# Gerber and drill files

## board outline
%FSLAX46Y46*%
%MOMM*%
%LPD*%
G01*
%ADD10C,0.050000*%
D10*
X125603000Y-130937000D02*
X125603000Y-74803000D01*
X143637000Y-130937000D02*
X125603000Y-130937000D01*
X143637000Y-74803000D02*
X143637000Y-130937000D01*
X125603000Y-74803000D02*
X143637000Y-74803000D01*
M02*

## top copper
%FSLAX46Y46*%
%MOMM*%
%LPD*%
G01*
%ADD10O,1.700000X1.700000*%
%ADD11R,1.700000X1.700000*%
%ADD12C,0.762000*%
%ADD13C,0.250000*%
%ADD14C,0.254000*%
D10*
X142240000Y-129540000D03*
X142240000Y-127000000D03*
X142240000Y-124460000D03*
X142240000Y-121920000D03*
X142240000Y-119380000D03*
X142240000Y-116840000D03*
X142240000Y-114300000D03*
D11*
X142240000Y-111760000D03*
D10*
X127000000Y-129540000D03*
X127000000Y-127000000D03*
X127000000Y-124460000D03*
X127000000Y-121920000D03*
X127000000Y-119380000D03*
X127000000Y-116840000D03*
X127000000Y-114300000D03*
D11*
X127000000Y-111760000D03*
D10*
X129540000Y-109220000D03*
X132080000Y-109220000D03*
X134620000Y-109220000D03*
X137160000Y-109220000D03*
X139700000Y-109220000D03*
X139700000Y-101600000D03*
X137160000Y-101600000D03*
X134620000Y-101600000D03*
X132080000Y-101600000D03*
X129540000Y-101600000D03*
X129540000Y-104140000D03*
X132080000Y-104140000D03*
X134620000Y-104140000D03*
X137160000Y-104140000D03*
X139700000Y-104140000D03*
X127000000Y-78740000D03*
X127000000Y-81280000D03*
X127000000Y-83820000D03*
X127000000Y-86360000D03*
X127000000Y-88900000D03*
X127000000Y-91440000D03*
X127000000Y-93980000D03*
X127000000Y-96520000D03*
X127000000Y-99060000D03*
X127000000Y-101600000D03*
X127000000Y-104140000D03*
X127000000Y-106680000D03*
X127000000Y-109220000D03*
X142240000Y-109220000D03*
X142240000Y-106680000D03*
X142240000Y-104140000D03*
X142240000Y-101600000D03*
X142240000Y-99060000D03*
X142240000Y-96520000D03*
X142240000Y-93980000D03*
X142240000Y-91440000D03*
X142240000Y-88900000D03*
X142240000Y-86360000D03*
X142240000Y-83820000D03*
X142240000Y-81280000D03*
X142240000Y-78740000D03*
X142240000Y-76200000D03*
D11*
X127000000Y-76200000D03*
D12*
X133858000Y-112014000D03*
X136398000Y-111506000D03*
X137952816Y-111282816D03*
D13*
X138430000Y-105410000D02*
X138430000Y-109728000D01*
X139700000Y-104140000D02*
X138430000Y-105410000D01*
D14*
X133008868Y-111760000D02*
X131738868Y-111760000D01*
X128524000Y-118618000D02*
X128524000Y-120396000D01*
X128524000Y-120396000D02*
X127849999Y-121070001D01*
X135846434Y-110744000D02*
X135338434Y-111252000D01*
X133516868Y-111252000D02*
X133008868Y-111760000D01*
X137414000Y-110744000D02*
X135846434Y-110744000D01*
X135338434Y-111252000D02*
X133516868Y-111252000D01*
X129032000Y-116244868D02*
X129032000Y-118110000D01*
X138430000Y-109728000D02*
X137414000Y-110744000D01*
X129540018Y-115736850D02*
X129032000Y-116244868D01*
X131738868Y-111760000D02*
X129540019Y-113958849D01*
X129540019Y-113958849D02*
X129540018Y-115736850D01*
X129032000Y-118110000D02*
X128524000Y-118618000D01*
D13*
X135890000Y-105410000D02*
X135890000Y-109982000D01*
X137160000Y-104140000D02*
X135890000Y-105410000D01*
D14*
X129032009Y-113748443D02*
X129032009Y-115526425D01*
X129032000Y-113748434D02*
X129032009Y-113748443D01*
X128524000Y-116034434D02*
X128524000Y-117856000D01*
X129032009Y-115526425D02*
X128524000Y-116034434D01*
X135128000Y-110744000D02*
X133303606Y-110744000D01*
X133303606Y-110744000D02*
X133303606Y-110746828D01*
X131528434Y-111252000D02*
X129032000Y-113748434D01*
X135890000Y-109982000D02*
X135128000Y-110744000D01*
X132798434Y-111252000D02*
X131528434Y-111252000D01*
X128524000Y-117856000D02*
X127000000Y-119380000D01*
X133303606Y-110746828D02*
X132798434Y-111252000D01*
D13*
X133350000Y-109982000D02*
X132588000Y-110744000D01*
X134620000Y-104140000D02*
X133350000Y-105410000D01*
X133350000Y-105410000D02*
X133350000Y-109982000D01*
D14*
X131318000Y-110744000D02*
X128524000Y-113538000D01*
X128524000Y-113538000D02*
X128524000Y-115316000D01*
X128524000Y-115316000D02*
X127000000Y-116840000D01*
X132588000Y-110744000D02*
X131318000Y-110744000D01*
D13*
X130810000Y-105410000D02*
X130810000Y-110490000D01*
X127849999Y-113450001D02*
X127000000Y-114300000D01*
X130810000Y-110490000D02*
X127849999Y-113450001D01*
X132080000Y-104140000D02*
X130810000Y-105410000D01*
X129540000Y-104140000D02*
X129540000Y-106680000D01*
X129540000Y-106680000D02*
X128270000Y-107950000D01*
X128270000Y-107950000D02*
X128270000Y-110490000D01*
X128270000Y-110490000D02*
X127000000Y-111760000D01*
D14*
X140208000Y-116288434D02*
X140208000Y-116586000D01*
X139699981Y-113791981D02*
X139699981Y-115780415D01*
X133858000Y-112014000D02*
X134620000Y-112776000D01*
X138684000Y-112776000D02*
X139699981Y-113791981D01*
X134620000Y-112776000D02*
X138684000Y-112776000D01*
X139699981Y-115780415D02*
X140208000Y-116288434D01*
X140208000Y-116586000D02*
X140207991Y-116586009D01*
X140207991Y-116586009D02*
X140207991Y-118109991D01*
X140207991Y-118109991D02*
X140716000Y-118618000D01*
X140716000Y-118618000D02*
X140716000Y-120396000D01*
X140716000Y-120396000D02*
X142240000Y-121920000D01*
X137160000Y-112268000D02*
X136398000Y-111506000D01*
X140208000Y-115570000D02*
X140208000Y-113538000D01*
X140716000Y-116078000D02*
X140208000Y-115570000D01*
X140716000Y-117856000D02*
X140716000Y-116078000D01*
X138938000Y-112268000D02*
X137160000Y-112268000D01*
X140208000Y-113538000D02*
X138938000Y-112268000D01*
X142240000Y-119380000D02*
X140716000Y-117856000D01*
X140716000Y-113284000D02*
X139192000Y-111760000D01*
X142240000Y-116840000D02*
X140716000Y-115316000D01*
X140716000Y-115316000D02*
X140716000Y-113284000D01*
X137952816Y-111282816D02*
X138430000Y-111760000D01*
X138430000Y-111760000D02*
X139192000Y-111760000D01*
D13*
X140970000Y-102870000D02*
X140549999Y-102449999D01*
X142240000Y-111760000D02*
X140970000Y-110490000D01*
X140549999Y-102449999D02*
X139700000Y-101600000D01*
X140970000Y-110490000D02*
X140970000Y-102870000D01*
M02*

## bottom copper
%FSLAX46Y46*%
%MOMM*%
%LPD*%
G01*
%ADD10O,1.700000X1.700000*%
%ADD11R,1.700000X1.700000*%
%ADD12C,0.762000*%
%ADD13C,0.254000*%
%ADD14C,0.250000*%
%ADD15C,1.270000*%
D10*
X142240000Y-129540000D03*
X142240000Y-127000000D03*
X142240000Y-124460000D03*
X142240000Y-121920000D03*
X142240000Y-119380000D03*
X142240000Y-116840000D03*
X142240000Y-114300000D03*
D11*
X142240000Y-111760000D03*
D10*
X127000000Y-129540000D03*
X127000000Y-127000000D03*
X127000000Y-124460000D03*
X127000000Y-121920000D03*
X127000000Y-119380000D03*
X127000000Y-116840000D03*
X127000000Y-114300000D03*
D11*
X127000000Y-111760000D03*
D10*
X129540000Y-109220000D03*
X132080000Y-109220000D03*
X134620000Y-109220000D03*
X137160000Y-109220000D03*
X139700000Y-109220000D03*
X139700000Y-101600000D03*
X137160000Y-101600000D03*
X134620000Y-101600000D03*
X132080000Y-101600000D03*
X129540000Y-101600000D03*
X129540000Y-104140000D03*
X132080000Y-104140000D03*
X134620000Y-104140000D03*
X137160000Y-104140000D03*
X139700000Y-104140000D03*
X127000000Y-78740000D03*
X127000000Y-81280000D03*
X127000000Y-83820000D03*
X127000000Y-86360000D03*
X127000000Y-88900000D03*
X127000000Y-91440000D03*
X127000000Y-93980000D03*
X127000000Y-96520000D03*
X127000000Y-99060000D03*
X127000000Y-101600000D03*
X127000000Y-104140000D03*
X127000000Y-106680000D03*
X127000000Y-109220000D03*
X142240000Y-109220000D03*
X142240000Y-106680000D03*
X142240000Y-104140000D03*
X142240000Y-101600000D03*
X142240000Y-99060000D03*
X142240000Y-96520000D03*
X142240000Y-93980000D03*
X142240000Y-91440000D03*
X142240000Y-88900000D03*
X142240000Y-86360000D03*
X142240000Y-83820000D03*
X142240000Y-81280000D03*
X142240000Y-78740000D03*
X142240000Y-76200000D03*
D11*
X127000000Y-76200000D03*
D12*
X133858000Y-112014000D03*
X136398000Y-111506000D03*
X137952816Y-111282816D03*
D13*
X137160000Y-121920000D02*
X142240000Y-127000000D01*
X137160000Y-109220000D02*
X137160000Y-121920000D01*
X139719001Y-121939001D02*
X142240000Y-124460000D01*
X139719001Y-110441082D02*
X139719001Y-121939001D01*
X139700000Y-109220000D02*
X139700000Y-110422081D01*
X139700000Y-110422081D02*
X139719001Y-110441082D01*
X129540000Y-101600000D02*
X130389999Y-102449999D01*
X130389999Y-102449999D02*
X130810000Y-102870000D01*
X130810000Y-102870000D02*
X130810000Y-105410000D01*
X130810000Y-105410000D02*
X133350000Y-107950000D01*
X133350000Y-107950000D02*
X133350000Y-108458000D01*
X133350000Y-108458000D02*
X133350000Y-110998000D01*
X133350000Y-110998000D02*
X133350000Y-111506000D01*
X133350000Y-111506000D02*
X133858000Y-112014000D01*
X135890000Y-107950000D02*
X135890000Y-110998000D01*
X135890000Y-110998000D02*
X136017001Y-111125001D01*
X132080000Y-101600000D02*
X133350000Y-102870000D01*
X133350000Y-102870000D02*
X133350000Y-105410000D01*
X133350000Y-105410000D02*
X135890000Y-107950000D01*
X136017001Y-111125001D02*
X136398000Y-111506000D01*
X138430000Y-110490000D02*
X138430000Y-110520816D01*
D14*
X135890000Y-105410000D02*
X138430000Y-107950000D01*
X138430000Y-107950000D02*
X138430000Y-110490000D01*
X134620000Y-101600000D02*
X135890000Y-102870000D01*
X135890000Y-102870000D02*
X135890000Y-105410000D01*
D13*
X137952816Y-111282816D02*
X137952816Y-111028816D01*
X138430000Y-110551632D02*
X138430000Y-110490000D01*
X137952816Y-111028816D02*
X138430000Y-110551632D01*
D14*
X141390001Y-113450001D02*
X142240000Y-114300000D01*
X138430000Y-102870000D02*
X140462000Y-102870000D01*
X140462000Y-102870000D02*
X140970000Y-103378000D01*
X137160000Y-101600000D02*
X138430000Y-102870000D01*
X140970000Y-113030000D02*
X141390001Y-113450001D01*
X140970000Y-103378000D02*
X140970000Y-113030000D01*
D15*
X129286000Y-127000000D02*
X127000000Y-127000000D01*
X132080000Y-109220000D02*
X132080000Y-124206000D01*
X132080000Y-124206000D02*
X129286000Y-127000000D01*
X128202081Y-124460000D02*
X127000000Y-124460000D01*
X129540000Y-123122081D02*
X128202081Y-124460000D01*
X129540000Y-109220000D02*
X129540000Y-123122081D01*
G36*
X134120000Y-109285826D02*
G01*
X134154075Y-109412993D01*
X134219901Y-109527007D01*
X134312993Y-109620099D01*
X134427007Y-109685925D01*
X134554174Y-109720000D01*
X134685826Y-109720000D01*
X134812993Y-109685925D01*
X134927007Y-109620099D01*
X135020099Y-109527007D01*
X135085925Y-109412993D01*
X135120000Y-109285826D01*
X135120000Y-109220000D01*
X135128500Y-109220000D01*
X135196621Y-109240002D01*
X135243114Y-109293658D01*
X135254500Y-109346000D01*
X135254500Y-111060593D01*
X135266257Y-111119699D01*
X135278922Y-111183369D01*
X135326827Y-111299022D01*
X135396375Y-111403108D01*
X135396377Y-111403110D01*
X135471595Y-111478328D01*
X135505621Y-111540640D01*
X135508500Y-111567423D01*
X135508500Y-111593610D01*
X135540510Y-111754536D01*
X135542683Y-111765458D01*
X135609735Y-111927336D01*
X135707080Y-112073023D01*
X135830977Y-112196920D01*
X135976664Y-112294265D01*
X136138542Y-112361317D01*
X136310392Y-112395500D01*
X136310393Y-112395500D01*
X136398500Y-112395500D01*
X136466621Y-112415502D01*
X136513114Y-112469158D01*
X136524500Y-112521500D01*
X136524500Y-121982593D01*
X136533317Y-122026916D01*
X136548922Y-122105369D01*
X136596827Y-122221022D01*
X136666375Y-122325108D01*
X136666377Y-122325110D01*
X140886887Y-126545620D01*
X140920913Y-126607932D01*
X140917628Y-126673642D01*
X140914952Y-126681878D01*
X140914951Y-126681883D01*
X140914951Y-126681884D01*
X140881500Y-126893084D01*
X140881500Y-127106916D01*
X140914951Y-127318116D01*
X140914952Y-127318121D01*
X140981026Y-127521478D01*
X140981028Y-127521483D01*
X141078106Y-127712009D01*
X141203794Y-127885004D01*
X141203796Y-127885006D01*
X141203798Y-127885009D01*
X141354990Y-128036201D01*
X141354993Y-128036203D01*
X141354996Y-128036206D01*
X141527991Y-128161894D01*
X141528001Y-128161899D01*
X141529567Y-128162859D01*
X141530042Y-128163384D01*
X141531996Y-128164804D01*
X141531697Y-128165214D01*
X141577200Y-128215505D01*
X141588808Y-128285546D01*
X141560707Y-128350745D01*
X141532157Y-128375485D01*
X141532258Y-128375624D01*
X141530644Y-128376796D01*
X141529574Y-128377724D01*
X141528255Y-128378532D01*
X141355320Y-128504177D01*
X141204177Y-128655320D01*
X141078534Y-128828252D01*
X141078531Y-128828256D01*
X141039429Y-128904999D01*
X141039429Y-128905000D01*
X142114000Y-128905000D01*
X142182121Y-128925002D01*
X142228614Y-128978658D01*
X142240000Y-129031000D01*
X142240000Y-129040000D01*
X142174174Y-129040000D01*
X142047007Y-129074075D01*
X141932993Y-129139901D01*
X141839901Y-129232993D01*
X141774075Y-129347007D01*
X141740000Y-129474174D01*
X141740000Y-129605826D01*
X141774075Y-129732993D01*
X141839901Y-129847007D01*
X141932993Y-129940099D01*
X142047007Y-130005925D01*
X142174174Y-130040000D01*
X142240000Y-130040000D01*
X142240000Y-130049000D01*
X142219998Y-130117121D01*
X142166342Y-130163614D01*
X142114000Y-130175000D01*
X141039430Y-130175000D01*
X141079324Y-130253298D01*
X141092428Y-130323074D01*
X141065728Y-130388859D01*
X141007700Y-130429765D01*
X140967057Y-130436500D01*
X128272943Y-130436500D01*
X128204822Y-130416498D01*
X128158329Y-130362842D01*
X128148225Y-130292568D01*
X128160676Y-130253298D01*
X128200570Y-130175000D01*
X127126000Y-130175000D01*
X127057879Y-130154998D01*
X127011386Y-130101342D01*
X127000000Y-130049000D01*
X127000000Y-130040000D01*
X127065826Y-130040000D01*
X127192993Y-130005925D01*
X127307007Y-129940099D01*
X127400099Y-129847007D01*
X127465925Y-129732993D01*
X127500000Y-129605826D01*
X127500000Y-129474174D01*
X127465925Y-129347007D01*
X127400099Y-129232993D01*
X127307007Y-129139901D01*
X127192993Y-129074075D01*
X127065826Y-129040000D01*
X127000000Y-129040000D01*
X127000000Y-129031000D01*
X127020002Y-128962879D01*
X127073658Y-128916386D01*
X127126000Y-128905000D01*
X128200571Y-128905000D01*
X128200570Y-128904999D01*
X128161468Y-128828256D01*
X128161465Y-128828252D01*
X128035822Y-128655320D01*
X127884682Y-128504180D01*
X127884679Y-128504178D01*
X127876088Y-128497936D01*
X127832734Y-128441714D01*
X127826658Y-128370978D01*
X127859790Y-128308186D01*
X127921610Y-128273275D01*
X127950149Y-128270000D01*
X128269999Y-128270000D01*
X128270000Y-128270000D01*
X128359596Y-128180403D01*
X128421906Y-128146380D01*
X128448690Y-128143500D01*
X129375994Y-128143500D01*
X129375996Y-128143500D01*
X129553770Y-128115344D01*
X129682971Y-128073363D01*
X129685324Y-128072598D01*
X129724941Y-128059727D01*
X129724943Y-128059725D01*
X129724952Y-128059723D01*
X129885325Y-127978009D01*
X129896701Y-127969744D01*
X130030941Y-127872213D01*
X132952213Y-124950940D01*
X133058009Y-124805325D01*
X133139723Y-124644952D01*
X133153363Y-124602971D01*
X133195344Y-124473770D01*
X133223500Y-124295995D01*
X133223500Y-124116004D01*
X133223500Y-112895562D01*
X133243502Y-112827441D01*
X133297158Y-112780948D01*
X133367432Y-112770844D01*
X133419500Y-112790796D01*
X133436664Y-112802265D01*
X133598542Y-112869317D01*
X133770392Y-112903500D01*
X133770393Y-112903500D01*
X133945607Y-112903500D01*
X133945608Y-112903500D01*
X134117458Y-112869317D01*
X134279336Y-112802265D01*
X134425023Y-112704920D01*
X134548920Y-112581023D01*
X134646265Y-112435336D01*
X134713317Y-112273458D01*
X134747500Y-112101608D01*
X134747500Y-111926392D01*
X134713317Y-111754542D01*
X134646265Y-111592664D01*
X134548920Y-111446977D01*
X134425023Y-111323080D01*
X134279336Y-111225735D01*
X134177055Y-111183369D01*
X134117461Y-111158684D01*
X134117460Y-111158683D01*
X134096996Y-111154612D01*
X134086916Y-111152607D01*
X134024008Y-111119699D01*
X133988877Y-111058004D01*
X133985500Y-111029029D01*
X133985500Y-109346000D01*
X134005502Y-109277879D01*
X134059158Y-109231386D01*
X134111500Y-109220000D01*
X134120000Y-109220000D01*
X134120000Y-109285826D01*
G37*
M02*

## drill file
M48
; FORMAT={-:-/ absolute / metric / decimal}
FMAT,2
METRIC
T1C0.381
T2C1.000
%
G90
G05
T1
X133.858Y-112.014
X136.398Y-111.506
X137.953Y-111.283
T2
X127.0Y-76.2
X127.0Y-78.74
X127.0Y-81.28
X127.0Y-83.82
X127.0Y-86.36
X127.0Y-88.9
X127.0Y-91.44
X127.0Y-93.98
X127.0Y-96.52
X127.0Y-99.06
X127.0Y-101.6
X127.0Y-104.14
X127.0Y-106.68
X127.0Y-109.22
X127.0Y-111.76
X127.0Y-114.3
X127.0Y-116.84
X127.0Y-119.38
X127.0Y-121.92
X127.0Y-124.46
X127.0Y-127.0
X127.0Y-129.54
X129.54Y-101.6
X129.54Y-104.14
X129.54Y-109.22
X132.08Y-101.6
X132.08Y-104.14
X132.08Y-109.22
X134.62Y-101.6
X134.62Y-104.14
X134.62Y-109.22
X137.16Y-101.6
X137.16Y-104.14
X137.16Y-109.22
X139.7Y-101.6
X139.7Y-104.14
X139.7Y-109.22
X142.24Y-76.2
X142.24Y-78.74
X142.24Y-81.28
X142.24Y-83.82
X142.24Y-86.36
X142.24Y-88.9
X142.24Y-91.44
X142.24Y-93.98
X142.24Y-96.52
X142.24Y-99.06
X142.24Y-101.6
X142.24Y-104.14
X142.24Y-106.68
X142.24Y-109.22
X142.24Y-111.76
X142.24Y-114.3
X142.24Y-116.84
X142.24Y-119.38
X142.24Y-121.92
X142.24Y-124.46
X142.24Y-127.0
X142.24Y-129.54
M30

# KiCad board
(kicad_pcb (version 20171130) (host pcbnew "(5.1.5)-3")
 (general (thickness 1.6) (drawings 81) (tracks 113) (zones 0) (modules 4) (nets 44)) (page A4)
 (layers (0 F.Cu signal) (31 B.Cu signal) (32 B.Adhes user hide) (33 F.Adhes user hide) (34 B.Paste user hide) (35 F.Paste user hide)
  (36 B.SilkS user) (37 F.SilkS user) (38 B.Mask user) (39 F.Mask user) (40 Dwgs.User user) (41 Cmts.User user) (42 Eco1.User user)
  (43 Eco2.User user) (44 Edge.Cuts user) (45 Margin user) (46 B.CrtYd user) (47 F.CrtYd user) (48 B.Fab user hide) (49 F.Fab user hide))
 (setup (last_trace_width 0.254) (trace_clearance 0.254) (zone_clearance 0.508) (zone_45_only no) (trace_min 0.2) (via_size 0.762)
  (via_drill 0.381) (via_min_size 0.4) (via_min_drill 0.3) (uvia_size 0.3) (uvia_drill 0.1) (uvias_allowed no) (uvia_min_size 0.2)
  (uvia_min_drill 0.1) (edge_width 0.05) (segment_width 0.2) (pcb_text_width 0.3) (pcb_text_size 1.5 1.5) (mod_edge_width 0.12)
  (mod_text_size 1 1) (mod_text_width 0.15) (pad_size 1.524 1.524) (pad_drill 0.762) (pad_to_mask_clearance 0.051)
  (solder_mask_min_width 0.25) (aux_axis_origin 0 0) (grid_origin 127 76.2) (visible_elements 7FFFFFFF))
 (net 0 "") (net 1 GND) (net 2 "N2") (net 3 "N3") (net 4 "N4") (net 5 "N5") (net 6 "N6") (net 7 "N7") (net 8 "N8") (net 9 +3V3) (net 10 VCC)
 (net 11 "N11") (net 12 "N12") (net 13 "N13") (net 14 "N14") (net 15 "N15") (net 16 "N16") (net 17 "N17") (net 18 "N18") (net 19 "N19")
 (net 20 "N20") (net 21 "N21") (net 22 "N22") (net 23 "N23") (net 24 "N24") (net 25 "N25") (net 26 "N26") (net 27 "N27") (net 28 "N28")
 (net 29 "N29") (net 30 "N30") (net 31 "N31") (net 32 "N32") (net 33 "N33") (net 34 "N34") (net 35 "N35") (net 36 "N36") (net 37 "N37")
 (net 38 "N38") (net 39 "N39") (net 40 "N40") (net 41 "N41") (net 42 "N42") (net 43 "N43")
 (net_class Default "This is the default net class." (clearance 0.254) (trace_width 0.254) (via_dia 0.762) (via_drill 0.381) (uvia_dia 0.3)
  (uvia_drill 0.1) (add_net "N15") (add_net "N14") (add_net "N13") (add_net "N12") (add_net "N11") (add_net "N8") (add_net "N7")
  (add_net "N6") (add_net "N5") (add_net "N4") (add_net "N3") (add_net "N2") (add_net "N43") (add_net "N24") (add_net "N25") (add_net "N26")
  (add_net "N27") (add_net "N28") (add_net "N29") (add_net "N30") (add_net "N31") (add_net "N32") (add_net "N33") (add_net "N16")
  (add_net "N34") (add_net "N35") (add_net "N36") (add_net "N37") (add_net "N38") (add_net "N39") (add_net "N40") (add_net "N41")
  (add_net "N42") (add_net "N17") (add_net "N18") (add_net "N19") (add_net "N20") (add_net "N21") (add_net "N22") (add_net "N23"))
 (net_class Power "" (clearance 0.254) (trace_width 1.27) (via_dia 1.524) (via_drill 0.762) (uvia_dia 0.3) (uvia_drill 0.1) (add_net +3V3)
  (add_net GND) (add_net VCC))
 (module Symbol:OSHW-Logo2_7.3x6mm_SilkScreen (layer F.Cu) (at 134.62 116.84)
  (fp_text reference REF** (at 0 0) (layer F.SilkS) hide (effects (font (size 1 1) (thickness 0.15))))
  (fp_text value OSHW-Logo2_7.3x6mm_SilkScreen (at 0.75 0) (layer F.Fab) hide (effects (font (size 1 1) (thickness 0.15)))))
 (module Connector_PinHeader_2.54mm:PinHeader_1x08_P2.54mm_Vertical (layer B.Cu) (at 142.24 111.76 180)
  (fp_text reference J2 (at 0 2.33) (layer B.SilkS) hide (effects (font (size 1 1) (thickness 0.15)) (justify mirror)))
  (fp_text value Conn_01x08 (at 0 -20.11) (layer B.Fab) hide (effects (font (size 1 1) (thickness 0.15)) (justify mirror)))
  (pad 8 thru_hole oval (at 0 -17.78 180) (size 1.7 1.7) (drill 1) (layers *.Cu *.Mask) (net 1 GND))
  (pad 7 thru_hole oval (at 0 -15.24 180) (size 1.7 1.7) (drill 1) (layers *.Cu *.Mask) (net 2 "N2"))
  (pad 6 thru_hole oval (at 0 -12.7 180) (size 1.7 1.7) (drill 1) (layers *.Cu *.Mask) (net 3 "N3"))
  (pad 5 thru_hole oval (at 0 -10.16 180) (size 1.7 1.7) (drill 1) (layers *.Cu *.Mask) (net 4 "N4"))
  (pad 4 thru_hole oval (at 0 -7.62 180) (size 1.7 1.7) (drill 1) (layers *.Cu *.Mask) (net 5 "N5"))
  (pad 3 thru_hole oval (at 0 -5.08 180) (size 1.7 1.7) (drill 1) (layers *.Cu *.Mask) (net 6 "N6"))
  (pad 2 thru_hole oval (at 0 -2.54 180) (size 1.7 1.7) (drill 1) (layers *.Cu *.Mask) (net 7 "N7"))
  (pad 1 thru_hole rect (at 0 0 180) (size 1.7 1.7) (drill 1) (layers *.Cu *.Mask) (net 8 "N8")))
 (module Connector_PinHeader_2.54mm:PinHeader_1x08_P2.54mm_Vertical (layer B.Cu) (at 127 111.76 180)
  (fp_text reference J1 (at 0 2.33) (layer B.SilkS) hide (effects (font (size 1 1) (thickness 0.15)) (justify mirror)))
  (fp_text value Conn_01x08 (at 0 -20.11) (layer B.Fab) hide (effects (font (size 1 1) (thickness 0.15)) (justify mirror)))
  (pad 8 thru_hole oval (at 0 -17.78 180) (size 1.7 1.7) (drill 1) (layers *.Cu *.Mask) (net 1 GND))
  (pad 7 thru_hole oval (at 0 -15.24 180) (size 1.7 1.7) (drill 1) (layers *.Cu *.Mask) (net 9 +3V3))
  (pad 6 thru_hole oval (at 0 -12.7 180) (size 1.7 1.7) (drill 1) (layers *.Cu *.Mask) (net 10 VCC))
  (pad 5 thru_hole oval (at 0 -10.16 180) (size 1.7 1.7) (drill 1) (layers *.Cu *.Mask) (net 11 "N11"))
  (pad 4 thru_hole oval (at 0 -7.62 180) (size 1.7 1.7) (drill 1) (layers *.Cu *.Mask) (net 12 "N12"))
  (pad 3 thru_hole oval (at 0 -5.08 180) (size 1.7 1.7) (drill 1) (layers *.Cu *.Mask) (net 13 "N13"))
  (pad 2 thru_hole oval (at 0 -2.54 180) (size 1.7 1.7) (drill 1) (layers *.Cu *.Mask) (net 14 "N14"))
  (pad 1 thru_hole rect (at 0 0 180) (size 1.7 1.7) (drill 1) (layers *.Cu *.Mask) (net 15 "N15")))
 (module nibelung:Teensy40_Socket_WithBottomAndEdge (layer F.Cu) (at 134.62 76.2)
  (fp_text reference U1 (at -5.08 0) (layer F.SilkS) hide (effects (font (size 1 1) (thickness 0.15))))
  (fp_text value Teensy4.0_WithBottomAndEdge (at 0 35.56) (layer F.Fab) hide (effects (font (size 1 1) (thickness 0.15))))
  (pad 43 thru_hole oval (at -5.08 33.02) (size 1.7 1.7) (drill 1) (layers *.Cu *.Mask) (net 10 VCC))
  (pad 42 thru_hole oval (at -2.54 33.02) (size 1.7 1.7) (drill 1) (layers *.Cu *.Mask) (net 9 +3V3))
  (pad 41 thru_hole oval (at 0 33.02) (size 1.7 1.7) (drill 1) (layers *.Cu *.Mask) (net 1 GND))
  (pad 40 thru_hole oval (at 2.54 33.02) (size 1.7 1.7) (drill 1) (layers *.Cu *.Mask) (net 2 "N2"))
  (pad 39 thru_hole oval (at 5.08 33.02) (size 1.7 1.7) (drill 1) (layers *.Cu *.Mask) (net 3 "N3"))
  (pad 38 thru_hole oval (at 5.08 25.4) (size 1.7 1.7) (drill 1) (layers *.Cu *.Mask) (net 8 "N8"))
  (pad 37 thru_hole oval (at 2.54 25.4) (size 1.7 1.7) (drill 1) (layers *.Cu *.Mask) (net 7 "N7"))
  (pad 36 thru_hole oval (at 0 25.4) (size 1.7 1.7) (drill 1) (layers *.Cu *.Mask) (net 6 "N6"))
  (pad 35 thru_hole oval (at -2.54 25.4) (size 1.7 1.7) (drill 1) (layers *.Cu *.Mask) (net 5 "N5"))
  (pad 34 thru_hole oval (at -5.08 25.4) (size 1.7 1.7) (drill 1) (layers *.Cu *.Mask) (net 4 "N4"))
  (pad 33 thru_hole oval (at -5.08 27.94) (size 1.7 1.7) (drill 1) (layers *.Cu *.Mask) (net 15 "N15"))
  (pad 32 thru_hole oval (at -2.54 27.94) (size 1.7 1.7) (drill 1) (layers *.Cu *.Mask) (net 14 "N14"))
  (pad 31 thru_hole oval (at 0 27.94) (size 1.7 1.7) (drill 1) (layers *.Cu *.Mask) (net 13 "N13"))
  (pad 30 thru_hole oval (at 2.54 27.94) (size 1.7 1.7) (drill 1) (layers *.Cu *.Mask) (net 12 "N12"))
  (pad 29 thru_hole oval (at 5.08 27.94) (size 1.7 1.7) (drill 1) (layers *.Cu *.Mask) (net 11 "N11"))
  (pad 2 thru_hole oval (at -7.62 2.54) (size 1.7 1.7) (drill 1) (layers *.Cu *.Mask) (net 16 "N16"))
  (pad 3 thru_hole oval (at -7.62 5.08) (size 1.7 1.7) (drill 1) (layers *.Cu *.Mask) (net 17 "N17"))
  (pad 4 thru_hole oval (at -7.62 7.62) (size 1.7 1.7) (drill 1) (layers *.Cu *.Mask) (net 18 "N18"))
  (pad 5 thru_hole oval (at -7.62 10.16) (size 1.7 1.7) (drill 1) (layers *.Cu *.Mask) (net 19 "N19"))
  (pad 6 thru_hole oval (at -7.62 12.7) (size 1.7 1.7) (drill 1) (layers *.Cu *.Mask) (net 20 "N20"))
  (pad 7 thru_hole oval (at -7.62 15.24) (size 1.7 1.7) (drill 1) (layers *.Cu *.Mask) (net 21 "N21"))
  (pad 8 thru_hole oval (at -7.62 17.78) (size 1.7 1.7) (drill 1) (layers *.Cu *.Mask) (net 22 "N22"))
  (pad 9 thru_hole oval (at -7.62 20.32) (size 1.7 1.7) (drill 1) (layers *.Cu *.Mask) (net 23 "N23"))
  (pad 10 thru_hole oval (at -7.62 22.86) (size 1.7 1.7) (drill 1) (layers *.Cu *.Mask) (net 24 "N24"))
  (pad 11 thru_hole oval (at -7.62 25.4) (size 1.7 1.7) (drill 1) (layers *.Cu *.Mask) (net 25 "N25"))
  (pad 12 thru_hole oval (at -7.62 27.94) (size 1.7 1.7) (drill 1) (layers *.Cu *.Mask) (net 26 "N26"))
  (pad 13 thru_hole oval (at -7.62 30.48) (size 1.7 1.7) (drill 1) (layers *.Cu *.Mask) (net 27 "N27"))
  (pad 14 thru_hole oval (at -7.62 33.02) (size 1.7 1.7) (drill 1) (layers *.Cu *.Mask) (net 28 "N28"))
  (pad 15 thru_hole oval (at 7.62 33.02) (size 1.7 1.7) (drill 1) (layers *.Cu *.Mask) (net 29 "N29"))
  (pad 16 thru_hole oval (at 7.62 30.48) (size 1.7 1.7) (drill 1) (layers *.Cu *.Mask) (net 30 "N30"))
  (pad 17 thru_hole oval (at 7.62 27.94) (size 1.7 1.7) (drill 1) (layers *.Cu *.Mask) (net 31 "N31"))
  (pad 18 thru_hole oval (at 7.62 25.4) (size 1.7 1.7) (drill 1) (layers *.Cu *.Mask) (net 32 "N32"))
  (pad 19 thru_hole oval (at 7.62 22.86) (size 1.7 1.7) (drill 1) (layers *.Cu *.Mask) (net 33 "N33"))
  (pad 20 thru_hole oval (at 7.62 20.32) (size 1.7 1.7) (drill 1) (layers *.Cu *.Mask) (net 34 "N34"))
  (pad 21 thru_hole oval (at 7.62 17.78) (size 1.7 1.7) (drill 1) (layers *.Cu *.Mask) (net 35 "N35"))
  (pad 22 thru_hole oval (at 7.62 15.24) (size 1.7 1.7) (drill 1) (layers *.Cu *.Mask) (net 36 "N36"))
  (pad 23 thru_hole oval (at 7.62 12.7) (size 1.7 1.7) (drill 1) (layers *.Cu *.Mask) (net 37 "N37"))
  (pad 24 thru_hole oval (at 7.62 10.16) (size 1.7 1.7) (drill 1) (layers *.Cu *.Mask) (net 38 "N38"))
  (pad 25 thru_hole oval (at 7.62 7.62) (size 1.7 1.7) (drill 1) (layers *.Cu *.Mask) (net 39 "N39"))
  (pad 26 thru_hole oval (at 7.62 5.08) (size 1.7 1.7) (drill 1) (layers *.Cu *.Mask) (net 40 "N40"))
  (pad 27 thru_hole oval (at 7.62 2.54) (size 1.7 1.7) (drill 1) (layers *.Cu *.Mask) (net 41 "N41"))
  (pad 28 thru_hole oval (at 7.62 0) (size 1.7 1.7) (drill 1) (layers *.Cu *.Mask) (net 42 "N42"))
  (pad 1 thru_hole rect (at -7.62 0) (size 1.7 1.7) (drill 1) (layers *.Cu *.Mask) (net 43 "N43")))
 (gr_line (start 125.603 130.937) (end 125.603 74.803) (layer Edge.Cuts) (width 0.05))
 (gr_line (start 143.637 130.937) (end 125.603 130.937) (layer Edge.Cuts) (width 0.05))
 (gr_line (start 143.637 74.803) (end 143.637 130.937) (layer Edge.Cuts) (width 0.05))
 (gr_line (start 125.603 74.803) (end 143.637 74.803) (layer Edge.Cuts) (width 0.05))
 (segment (start 138.43 105.41) (end 138.43 109.728) (width 0.25) (layer F.Cu) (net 11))
 (segment (start 139.7 104.14) (end 138.43 105.41) (width 0.25) (layer F.Cu) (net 11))
 (segment (start 133.008868 111.76) (end 131.738868 111.76) (width 0.254) (layer F.Cu) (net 11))
 (segment (start 128.524 118.618) (end 128.524 120.396) (width 0.254) (layer F.Cu) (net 11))
 (segment (start 128.524 120.396) (end 127.849999 121.070001) (width 0.254) (layer F.Cu) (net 11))
 (segment (start 135.846434 110.744) (end 135.338434 111.252) (width 0.254) (layer F.Cu) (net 11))
 (segment (start 133.516868 111.252) (end 133.008868 111.76) (width 0.254) (layer F.Cu) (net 11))
 (segment (start 137.414 110.744) (end 135.846434 110.744) (width 0.254) (layer F.Cu) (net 11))
 (segment (start 135.338434 111.252) (end 133.516868 111.252) (width 0.254) (layer F.Cu) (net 11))
 (segment (start 129.032 116.244868) (end 129.032 118.11) (width 0.254) (layer F.Cu) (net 11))
 (segment (start 138.43 109.728) (end 137.414 110.744) (width 0.254) (layer F.Cu) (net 11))
 (segment (start 129.540018 115.73685) (end 129.032 116.244868) (width 0.254) (layer F.Cu) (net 11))
 (segment (start 131.738868 111.76) (end 129.540019 113.958849) (width 0.254) (layer F.Cu) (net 11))
 (segment (start 129.540019 113.958849) (end 129.540018 115.73685) (width 0.254) (layer F.Cu) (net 11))
 (segment (start 129.032 118.11) (end 128.524 118.618) (width 0.254) (layer F.Cu) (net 11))
 (segment (start 135.89 105.41) (end 135.89 109.982) (width 0.25) (layer F.Cu) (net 12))
 (segment (start 137.16 104.14) (end 135.89 105.41) (width 0.25) (layer F.Cu) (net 12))
 (segment (start 129.032009 113.748443) (end 129.032009 115.526425) (width 0.254) (layer F.Cu) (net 12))
 (segment (start 129.032 113.748434) (end 129.032009 113.748443) (width 0.254) (layer F.Cu) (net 12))
 (segment (start 128.524 116.034434) (end 128.524 117.856) (width 0.254) (layer F.Cu) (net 12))
 (segment (start 129.032009 115.526425) (end 128.524 116.034434) (width 0.254) (layer F.Cu) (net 12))
 (segment (start 135.128 110.744) (end 133.303606 110.744) (width 0.254) (layer F.Cu) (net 12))
 (segment (start 133.303606 110.744) (end 133.303606 110.746828) (width 0.254) (layer F.Cu) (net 12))
 (segment (start 131.528434 111.252) (end 129.032 113.748434) (width 0.254) (layer F.Cu) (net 12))
 (segment (start 135.89 109.982) (end 135.128 110.744) (width 0.254) (layer F.Cu) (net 12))
 (segment (start 132.798434 111.252) (end 131.528434 111.252) (width 0.254) (layer F.Cu) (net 12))
 (segment (start 128.524 117.856) (end 127 119.38) (width 0.254) (layer F.Cu) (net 12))
 (segment (start 133.303606 110.746828) (end 132.798434 111.252) (width 0.254) (layer F.Cu) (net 12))
 (segment (start 133.35 109.982) (end 132.588 110.744) (width 0.25) (layer F.Cu) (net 13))
 (segment (start 134.62 104.14) (end 133.35 105.41) (width 0.25) (layer F.Cu) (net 13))
 (segment (start 133.35 105.41) (end 133.35 109.982) (width 0.25) (layer F.Cu) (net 13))
 (segment (start 131.318 110.744) (end 128.524 113.538) (width 0.254) (layer F.Cu) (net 13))
 (segment (start 128.524 113.538) (end 128.524 115.316) (width 0.254) (layer F.Cu) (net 13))
 (segment (start 128.524 115.316) (end 127 116.84) (width 0.254) (layer F.Cu) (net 13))
 (segment (start 132.588 110.744) (end 131.318 110.744) (width 0.254) (layer F.Cu) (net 13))
 (segment (start 130.81 105.41) (end 130.81 110.49) (width 0.25) (layer F.Cu) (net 14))
 (segment (start 127.849999 113.450001) (end 127 114.3) (width 0.25) (layer F.Cu) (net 14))
 (segment (start 130.81 110.49) (end 127.849999 113.450001) (width 0.25) (layer F.Cu) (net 14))
 (segment (start 132.08 104.14) (end 130.81 105.41) (width 0.25) (layer F.Cu) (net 14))
 (segment (start 129.54 104.14) (end 129.54 106.68) (width 0.25) (layer F.Cu) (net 15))
 (segment (start 129.54 106.68) (end 128.27 107.95) (width 0.25) (layer F.Cu) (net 15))
 (segment (start 128.27 107.95) (end 128.27 110.49) (width 0.25) (layer F.Cu) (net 15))
 (segment (start 128.27 110.49) (end 127 111.76) (width 0.25) (layer F.Cu) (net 15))
 (segment (start 137.16 121.92) (end 142.24 127) (width 0.254) (layer B.Cu) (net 2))
 (segment (start 137.16 109.22) (end 137.16 121.92) (width 0.254) (layer B.Cu) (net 2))
 (segment (start 139.719001 121.939001) (end 142.24 124.46) (width 0.254) (layer B.Cu) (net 3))
 (segment (start 139.719001 110.441082) (end 139.719001 121.939001) (width 0.254) (layer B.Cu) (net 3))
 (segment (start 139.7 109.22) (end 139.7 110.422081) (width 0.254) (layer B.Cu) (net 3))
 (segment (start 139.7 110.422081) (end 139.719001 110.441082) (width 0.254) (layer B.Cu) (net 3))
 (segment (start 129.54 101.6) (end 130.389999 102.449999) (width 0.254) (layer B.Cu) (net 4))
 (segment (start 130.389999 102.449999) (end 130.81 102.87) (width 0.254) (layer B.Cu) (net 4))
 (segment (start 130.81 102.87) (end 130.81 105.41) (width 0.254) (layer B.Cu) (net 4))
 (segment (start 130.81 105.41) (end 133.35 107.95) (width 0.254) (layer B.Cu) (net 4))
 (segment (start 133.35 107.95) (end 133.35 108.458) (width 0.254) (layer B.Cu) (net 4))
 (segment (start 133.35 108.458) (end 133.35 110.998) (width 0.254) (layer B.Cu) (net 4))
 (via (at 133.858 112.014) (size 0.762) (drill 0.381) (layers F.Cu B.Cu) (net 4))
 (segment (start 133.35 110.998) (end 133.35 111.506) (width 0.254) (layer B.Cu) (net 4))
 (segment (start 133.35 111.506) (end 133.858 112.014) (width 0.254) (layer B.Cu) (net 4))
 (segment (start 140.208 116.288434) (end 140.208 116.586) (width 0.254) (layer F.Cu) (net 4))
 (segment (start 139.699981 113.791981) (end 139.699981 115.780415) (width 0.254) (layer F.Cu) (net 4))
 (segment (start 133.858 112.014) (end 134.62 112.776) (width 0.254) (layer F.Cu) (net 4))
 (segment (start 138.684 112.776) (end 139.699981 113.791981) (width 0.254) (layer F.Cu) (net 4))
 (segment (start 134.62 112.776) (end 138.684 112.776) (width 0.254) (layer F.Cu) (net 4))
 (segment (start 139.699981 115.780415) (end 140.208 116.288434) (width 0.254) (layer F.Cu) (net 4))
 (segment (start 140.208 116.586) (end 140.207991 116.586009) (width 0.254) (layer F.Cu) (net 4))
 (segment (start 140.207991 116.586009) (end 140.207991 118.109991) (width 0.254) (layer F.Cu) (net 4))
 (segment (start 140.207991 118.109991) (end 140.716 118.618) (width 0.254) (layer F.Cu) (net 4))
 (segment (start 140.716 118.618) (end 140.716 120.396) (width 0.254) (layer F.Cu) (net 4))
 (segment (start 140.716 120.396) (end 142.24 121.92) (width 0.254) (layer F.Cu) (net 4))
 (segment (start 135.89 107.95) (end 135.89 110.998) (width 0.254) (layer B.Cu) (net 5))
 (segment (start 135.89 110.998) (end 136.017001 111.125001) (width 0.254) (layer B.Cu) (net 5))
 (segment (start 132.08 101.6) (end 133.35 102.87) (width 0.254) (layer B.Cu) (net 5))
 (segment (start 133.35 102.87) (end 133.35 105.41) (width 0.254) (layer B.Cu) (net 5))
 (via (at 136.398 111.506) (size 0.762) (drill 0.381) (layers F.Cu B.Cu) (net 5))
 (segment (start 133.35 105.41) (end 135.89 107.95) (width 0.254) (layer B.Cu) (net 5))
 (segment (start 136.017001 111.125001) (end 136.398 111.506) (width 0.254) (layer B.Cu) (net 5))
 (segment (start 137.16 112.268) (end 136.398 111.506) (width 0.254) (layer F.Cu) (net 5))
 (segment (start 140.208 115.57) (end 140.208 113.538) (width 0.254) (layer F.Cu) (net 5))
 (segment (start 140.716 116.078) (end 140.208 115.57) (width 0.254) (layer F.Cu) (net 5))
 (segment (start 140.716 117.856) (end 140.716 116.078) (width 0.254) (layer F.Cu) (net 5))
 (segment (start 138.938 112.268) (end 137.16 112.268) (width 0.254) (layer F.Cu) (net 5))
 (segment (start 140.208 113.538) (end 138.938 112.268) (width 0.254) (layer F.Cu) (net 5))
 (segment (start 142.24 119.38) (end 140.716 117.856) (width 0.254) (layer F.Cu) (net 5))
 (segment (start 140.716 113.284) (end 139.192 111.76) (width 0.254) (layer F.Cu) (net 6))
 (segment (start 142.24 116.84) (end 140.716 115.316) (width 0.254) (layer F.Cu) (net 6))
 (segment (start 140.716 115.316) (end 140.716 113.284) (width 0.254) (layer F.Cu) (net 6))
 (via (at 137.952816 111.282816) (size 0.762) (drill 0.381) (layers F.Cu B.Cu) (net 6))
 (segment (start 137.952816 111.282816) (end 138.43 111.76) (width 0.254) (layer F.Cu) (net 6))
 (segment (start 138.43 111.76) (end 139.192 111.76) (width 0.254) (layer F.Cu) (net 6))
 (segment (start 138.43 110.49) (end 138.43 110.520816) (width 0.254) (layer B.Cu) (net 6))
 (segment (start 135.89 105.41) (end 138.43 107.95) (width 0.25) (layer B.Cu) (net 6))
 (segment (start 138.43 107.95) (end 138.43 110.49) (width 0.25) (layer B.Cu) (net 6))
 (segment (start 134.62 101.6) (end 135.89 102.87) (width 0.25) (layer B.Cu) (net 6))
 (segment (start 135.89 102.87) (end 135.89 105.41) (width 0.25) (layer B.Cu) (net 6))
 (segment (start 137.952816 111.282816) (end 137.952816 111.028816) (width 0.254) (layer B.Cu) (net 6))
 (segment (start 138.43 110.551632) (end 138.43 110.49) (width 0.254) (layer B.Cu) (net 6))
 (segment (start 137.952816 111.028816) (end 138.43 110.551632) (width 0.254) (layer B.Cu) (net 6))
 (segment (start 141.390001 113.450001) (end 142.24 114.3) (width 0.25) (layer B.Cu) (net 7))
 (segment (start 138.43 102.87) (end 140.462 102.87) (width 0.25) (layer B.Cu) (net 7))
 (segment (start 140.462 102.87) (end 140.97 103.378) (width 0.25) (layer B.Cu) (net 7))
 (segment (start 137.16 101.6) (end 138.43 102.87) (width 0.25) (layer B.Cu) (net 7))
 (segment (start 140.97 113.03) (end 141.390001 113.450001) (width 0.25) (layer B.Cu) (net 7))
 (segment (start 140.97 103.378) (end 140.97 113.03) (width 0.25) (layer B.Cu) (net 7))
 (segment (start 140.97 102.87) (end 140.549999 102.449999) (width 0.25) (layer F.Cu) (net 8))
 (segment (start 142.24 111.76) (end 140.97 110.49) (width 0.25) (layer F.Cu) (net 8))
 (segment (start 140.549999 102.449999) (end 139.7 101.6) (width 0.25) (layer F.Cu) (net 8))
 (segment (start 140.97 110.49) (end 140.97 102.87) (width 0.25) (layer F.Cu) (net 8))
 (segment (start 129.286 127) (end 127 127) (width 1.27) (layer B.Cu) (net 9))
 (segment (start 132.08 109.22) (end 132.08 124.206) (width 1.27) (layer B.Cu) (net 9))
 (segment (start 132.08 124.206) (end 129.286 127) (width 1.27) (layer B.Cu) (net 9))
 (segment (start 128.202081 124.46) (end 127 124.46) (width 1.27) (layer B.Cu) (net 10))
 (segment (start 129.54 123.122081) (end 128.202081 124.46) (width 1.27) (layer B.Cu) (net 10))
 (segment (start 129.54 109.22) (end 129.54 123.122081) (width 1.27) (layer B.Cu) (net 10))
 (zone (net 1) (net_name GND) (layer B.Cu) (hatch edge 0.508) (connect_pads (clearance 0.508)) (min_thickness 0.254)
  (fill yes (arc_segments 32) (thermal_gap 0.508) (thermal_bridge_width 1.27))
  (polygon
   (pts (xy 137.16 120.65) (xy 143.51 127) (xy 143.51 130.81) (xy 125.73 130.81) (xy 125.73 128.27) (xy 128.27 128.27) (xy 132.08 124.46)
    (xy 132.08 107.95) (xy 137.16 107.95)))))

